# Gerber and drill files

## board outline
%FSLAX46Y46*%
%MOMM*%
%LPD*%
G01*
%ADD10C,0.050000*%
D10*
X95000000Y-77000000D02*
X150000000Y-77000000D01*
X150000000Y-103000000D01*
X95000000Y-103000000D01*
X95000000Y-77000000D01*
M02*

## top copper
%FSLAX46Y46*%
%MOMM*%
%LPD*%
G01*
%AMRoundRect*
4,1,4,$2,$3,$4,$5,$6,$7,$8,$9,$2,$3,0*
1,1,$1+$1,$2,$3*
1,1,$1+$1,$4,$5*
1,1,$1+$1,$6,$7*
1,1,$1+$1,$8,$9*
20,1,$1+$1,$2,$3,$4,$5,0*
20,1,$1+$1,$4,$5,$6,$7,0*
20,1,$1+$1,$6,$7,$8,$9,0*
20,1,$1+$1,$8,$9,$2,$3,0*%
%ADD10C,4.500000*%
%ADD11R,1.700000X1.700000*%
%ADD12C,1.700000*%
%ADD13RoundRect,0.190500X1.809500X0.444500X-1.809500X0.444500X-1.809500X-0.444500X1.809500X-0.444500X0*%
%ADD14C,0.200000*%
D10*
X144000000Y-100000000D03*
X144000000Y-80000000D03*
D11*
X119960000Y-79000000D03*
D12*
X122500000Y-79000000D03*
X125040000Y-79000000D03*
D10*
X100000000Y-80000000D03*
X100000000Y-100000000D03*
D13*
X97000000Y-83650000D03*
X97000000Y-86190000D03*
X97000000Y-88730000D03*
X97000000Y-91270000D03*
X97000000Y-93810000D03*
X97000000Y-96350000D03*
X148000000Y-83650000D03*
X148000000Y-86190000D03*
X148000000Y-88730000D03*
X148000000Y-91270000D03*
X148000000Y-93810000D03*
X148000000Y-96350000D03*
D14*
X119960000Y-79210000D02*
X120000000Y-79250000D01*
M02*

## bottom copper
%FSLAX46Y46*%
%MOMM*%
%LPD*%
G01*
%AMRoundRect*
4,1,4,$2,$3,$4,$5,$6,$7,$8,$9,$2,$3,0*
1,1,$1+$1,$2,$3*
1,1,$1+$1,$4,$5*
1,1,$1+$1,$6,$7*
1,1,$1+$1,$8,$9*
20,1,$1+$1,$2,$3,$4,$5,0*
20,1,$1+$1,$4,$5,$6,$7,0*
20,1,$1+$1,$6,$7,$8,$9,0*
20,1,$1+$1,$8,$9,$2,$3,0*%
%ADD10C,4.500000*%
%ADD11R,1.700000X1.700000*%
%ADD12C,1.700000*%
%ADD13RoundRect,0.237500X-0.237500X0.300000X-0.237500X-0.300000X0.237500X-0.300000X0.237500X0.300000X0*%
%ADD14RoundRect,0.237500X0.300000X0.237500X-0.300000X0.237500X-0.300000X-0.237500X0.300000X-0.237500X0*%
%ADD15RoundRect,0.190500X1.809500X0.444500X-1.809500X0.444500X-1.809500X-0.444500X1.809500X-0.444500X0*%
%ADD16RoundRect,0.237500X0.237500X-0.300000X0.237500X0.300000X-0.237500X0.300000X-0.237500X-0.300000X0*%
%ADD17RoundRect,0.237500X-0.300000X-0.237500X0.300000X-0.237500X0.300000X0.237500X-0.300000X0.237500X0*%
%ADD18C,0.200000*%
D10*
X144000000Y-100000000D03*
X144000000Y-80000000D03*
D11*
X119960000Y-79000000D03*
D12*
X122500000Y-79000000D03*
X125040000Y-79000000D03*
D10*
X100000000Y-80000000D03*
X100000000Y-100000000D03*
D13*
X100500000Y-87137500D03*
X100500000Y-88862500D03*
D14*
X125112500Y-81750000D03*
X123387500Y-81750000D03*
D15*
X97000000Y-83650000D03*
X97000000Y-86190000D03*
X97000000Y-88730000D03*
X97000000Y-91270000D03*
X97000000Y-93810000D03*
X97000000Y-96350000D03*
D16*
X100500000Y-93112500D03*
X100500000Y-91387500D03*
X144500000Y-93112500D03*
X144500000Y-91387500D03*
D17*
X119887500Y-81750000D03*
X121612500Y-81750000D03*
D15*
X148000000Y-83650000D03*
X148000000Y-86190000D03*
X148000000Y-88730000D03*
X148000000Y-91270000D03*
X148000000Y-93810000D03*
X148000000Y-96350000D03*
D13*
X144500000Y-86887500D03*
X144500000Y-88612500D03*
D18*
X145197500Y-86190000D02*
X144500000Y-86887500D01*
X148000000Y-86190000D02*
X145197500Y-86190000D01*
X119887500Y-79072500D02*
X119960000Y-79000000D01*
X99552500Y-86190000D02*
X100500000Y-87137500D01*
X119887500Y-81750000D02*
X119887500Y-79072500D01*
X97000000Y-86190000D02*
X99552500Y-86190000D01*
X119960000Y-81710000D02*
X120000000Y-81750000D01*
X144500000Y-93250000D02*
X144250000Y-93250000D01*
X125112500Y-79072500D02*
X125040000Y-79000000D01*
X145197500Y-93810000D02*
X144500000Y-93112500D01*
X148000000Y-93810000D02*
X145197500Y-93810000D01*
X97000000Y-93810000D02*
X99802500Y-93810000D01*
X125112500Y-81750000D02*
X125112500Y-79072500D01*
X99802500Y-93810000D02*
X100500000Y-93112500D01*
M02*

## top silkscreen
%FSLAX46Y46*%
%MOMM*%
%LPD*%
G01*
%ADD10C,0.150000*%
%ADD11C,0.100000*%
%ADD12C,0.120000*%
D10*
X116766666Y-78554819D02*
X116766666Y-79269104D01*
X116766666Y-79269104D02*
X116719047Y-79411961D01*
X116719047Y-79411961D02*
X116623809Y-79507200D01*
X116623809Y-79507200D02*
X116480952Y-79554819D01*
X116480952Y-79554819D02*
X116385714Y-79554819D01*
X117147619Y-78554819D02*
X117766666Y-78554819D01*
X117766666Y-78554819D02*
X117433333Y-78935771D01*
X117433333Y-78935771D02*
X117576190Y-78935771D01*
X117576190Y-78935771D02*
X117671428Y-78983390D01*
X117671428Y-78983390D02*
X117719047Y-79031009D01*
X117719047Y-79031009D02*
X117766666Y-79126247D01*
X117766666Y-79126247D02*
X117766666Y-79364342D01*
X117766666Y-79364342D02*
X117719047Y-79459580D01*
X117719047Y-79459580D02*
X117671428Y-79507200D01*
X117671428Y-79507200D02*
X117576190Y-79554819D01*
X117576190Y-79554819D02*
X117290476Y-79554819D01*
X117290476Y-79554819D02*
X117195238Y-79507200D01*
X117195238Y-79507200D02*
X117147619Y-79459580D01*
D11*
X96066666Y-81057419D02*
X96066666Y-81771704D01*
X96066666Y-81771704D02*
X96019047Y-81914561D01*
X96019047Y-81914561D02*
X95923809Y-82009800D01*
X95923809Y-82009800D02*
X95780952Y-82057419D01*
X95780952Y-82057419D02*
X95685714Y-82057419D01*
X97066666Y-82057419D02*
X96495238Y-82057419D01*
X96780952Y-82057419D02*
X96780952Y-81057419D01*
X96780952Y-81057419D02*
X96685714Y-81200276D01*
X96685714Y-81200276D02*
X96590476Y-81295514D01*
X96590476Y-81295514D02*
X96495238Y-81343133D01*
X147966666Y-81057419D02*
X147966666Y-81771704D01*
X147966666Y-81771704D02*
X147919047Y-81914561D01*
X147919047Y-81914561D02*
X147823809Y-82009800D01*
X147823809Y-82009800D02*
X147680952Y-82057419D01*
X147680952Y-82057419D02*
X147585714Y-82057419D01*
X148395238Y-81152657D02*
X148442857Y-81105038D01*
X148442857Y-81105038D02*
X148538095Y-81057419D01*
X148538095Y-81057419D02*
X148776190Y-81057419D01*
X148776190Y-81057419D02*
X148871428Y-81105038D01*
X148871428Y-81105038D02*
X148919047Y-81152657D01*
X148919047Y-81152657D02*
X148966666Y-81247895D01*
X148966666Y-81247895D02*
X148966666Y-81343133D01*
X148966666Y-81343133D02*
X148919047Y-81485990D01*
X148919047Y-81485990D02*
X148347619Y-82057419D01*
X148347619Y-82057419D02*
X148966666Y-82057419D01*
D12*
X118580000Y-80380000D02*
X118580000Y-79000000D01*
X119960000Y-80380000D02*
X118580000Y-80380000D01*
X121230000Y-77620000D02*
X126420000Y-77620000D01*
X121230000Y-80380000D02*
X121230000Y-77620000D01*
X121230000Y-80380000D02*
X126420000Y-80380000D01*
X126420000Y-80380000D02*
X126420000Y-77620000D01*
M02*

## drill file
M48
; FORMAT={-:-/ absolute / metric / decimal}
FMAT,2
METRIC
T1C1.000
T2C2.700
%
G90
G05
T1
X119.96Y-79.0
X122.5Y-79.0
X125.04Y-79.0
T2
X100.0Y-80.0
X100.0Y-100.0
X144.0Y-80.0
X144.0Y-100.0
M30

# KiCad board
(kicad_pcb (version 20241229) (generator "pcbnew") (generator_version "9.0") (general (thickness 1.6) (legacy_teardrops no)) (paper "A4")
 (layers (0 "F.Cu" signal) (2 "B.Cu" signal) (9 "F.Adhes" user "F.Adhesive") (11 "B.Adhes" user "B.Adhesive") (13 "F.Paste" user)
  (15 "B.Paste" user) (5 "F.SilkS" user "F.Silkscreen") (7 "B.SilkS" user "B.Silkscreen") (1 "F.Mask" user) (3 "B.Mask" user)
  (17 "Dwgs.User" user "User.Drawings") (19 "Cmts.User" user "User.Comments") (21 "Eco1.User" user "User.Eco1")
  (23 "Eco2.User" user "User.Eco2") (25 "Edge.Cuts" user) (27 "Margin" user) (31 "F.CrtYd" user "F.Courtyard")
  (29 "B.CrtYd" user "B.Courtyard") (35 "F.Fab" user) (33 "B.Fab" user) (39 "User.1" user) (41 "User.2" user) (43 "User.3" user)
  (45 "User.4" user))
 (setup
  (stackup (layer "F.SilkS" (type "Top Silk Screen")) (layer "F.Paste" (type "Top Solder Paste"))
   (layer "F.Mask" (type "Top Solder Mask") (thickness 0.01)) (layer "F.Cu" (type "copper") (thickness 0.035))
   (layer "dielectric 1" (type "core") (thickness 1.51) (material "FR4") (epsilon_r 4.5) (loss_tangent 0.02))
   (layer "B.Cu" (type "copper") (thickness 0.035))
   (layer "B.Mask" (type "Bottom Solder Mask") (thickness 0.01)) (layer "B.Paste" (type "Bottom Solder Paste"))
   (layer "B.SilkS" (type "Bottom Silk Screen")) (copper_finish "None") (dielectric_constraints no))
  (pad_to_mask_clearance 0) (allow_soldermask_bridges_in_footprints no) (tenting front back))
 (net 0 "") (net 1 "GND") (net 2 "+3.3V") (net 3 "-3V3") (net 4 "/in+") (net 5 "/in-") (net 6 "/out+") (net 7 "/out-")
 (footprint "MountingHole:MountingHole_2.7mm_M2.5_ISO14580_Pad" (layer "F.Cu") (at 144 100)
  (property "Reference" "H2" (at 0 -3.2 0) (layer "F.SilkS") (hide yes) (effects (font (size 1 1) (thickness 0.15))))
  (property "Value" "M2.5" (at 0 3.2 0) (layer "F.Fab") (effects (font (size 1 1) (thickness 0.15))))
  (pad "1" thru_hole circle (at 0 0) (size 4.5 4.5) (drill 2.7) (layers "*.Cu" "*.Mask") (remove_unused_layers no) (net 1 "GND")
   (zone_connect 2)))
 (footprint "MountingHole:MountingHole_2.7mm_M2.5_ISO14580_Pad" (layer "F.Cu") (at 144 80)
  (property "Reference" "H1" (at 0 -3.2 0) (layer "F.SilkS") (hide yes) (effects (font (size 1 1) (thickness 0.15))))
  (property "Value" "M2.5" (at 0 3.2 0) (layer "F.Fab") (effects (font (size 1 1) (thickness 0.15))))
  (pad "1" thru_hole circle (at 0 0) (size 4.5 4.5) (drill 2.7) (layers "*.Cu" "*.Mask") (remove_unused_layers no) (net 1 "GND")
   (zone_connect 2)))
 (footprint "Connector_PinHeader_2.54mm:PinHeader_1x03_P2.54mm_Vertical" (layer "F.Cu") (at 119.96 79 90)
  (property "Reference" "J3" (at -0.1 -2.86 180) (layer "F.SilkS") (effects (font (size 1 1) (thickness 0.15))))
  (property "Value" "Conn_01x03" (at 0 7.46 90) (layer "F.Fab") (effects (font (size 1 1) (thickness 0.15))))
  (fp_line (start -1.38 -1.38) (end 0 -1.38) (stroke (width 0.12) (type solid)) (layer "F.SilkS"))
  (fp_line (start -1.38 0) (end -1.38 -1.38) (stroke (width 0.12) (type solid)) (layer "F.SilkS"))
  (fp_line (start 1.38 1.27) (end 1.38 6.46) (stroke (width 0.12) (type solid)) (layer "F.SilkS"))
  (fp_line (start -1.38 1.27) (end 1.38 1.27) (stroke (width 0.12) (type solid)) (layer "F.SilkS"))
  (fp_line (start -1.38 1.27) (end -1.38 6.46) (stroke (width 0.12) (type solid)) (layer "F.SilkS"))
  (fp_line (start -1.38 6.46) (end 1.38 6.46) (stroke (width 0.12) (type solid)) (layer "F.SilkS"))
  (pad "1" thru_hole rect (at 0 0 90) (size 1.7 1.7) (drill 1) (layers "*.Cu" "*.Mask") (remove_unused_layers no) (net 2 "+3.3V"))
  (pad "2" thru_hole circle (at 0 2.54 90) (size 1.7 1.7) (drill 1) (layers "*.Cu" "*.Mask") (remove_unused_layers no) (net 1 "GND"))
  (pad "3" thru_hole circle (at 0 5.08 90) (size 1.7 1.7) (drill 1) (layers "*.Cu" "*.Mask") (remove_unused_layers no) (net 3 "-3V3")))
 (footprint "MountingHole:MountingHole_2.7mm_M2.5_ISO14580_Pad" (layer "F.Cu") (at 100 80)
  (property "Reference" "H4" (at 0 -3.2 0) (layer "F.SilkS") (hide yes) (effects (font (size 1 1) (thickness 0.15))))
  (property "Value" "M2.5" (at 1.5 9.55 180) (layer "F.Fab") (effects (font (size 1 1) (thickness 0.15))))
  (pad "1" thru_hole circle (at 0 0) (size 4.5 4.5) (drill 2.7) (layers "*.Cu" "*.Mask") (remove_unused_layers no) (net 1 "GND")
   (zone_connect 2)))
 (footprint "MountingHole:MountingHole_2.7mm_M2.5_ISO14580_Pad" (layer "F.Cu") (at 100 100)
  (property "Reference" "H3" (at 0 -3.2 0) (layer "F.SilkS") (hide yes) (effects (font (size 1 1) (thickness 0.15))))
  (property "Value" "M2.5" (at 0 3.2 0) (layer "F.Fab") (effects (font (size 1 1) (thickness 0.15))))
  (pad "1" thru_hole circle (at 0 0) (size 4.5 4.5) (drill 2.7) (layers "*.Cu" "*.Mask") (remove_unused_layers no) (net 1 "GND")
   (zone_connect 2)))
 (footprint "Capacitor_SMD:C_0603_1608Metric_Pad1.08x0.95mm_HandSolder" (layer "B.Cu") (at 100.5 88 -90)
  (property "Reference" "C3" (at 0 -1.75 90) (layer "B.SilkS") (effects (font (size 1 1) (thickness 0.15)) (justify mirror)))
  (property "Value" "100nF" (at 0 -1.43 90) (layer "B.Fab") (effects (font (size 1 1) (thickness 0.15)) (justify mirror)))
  (pad "1" smd roundrect (at -0.8625 0 270) (size 1.075 0.95) (layers "B.Cu" "B.Mask" "B.Paste") (roundrect_rratio 0.25) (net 2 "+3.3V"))
  (pad "2" smd roundrect (at 0.8625 0 270) (size 1.075 0.95) (layers "B.Cu" "B.Mask" "B.Paste") (roundrect_rratio 0.25) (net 1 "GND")))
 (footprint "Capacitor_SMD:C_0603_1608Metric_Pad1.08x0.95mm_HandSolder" (layer "B.Cu") (at 124.25 81.75 180)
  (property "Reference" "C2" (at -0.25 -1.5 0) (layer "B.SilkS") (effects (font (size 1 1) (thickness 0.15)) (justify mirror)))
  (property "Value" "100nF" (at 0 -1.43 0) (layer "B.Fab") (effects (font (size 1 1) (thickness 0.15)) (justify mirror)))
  (pad "1" smd roundrect (at -0.8625 0 180) (size 1.075 0.95) (layers "B.Cu" "B.Mask" "B.Paste") (roundrect_rratio 0.25) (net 3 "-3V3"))
  (pad "2" smd roundrect (at 0.8625 0 180) (size 1.075 0.95) (layers "B.Cu" "B.Mask" "B.Paste") (roundrect_rratio 0.25) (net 1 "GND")))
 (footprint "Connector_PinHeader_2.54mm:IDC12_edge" (layer "B.Cu") (at 97 83.65 180)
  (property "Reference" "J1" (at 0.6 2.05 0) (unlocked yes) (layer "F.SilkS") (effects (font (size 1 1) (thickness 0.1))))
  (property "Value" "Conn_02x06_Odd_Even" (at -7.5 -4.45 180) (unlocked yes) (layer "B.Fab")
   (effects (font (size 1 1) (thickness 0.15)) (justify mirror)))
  (pad "1" smd roundrect (at 0 0 180) (size 4 1.27) (layers "B.Cu" "B.Mask" "B.Paste") (roundrect_rratio 0.15) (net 1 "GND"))
  (pad "2" smd roundrect (at 0 0 180) (size 4 1.27) (layers "F.Cu" "F.Mask" "F.Paste") (roundrect_rratio 0.15) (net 1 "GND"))
  (pad "3" smd roundrect (at 0 -2.54 180) (size 4 1.27) (layers "B.Cu" "B.Mask" "B.Paste") (roundrect_rratio 0.15) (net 2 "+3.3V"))
  (pad "4" smd roundrect (at 0 -2.54 180) (size 4 1.27) (layers "F.Cu" "F.Mask" "F.Paste") (roundrect_rratio 0.15) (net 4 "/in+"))
  (pad "5" smd roundrect (at 0 -5.08 180) (size 4 1.27) (layers "B.Cu" "B.Mask" "B.Paste") (roundrect_rratio 0.15) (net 1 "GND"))
  (pad "6" smd roundrect (at 0 -5.08 180) (size 4 1.27) (layers "F.Cu" "F.Mask" "F.Paste") (roundrect_rratio 0.15) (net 1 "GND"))
  (pad "7" smd roundrect (at 0 -7.62 180) (size 4 1.27) (layers "B.Cu" "B.Mask" "B.Paste") (roundrect_rratio 0.15) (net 1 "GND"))
  (pad "8" smd roundrect (at 0 -7.62 180) (size 4 1.27) (layers "F.Cu" "F.Mask" "F.Paste") (roundrect_rratio 0.15) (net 1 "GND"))
  (pad "9" smd roundrect (at 0 -10.16 180) (size 4 1.27) (layers "B.Cu" "B.Mask" "B.Paste") (roundrect_rratio 0.15) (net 3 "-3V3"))
  (pad "10" smd roundrect (at 0 -10.16 180) (size 4 1.27) (layers "F.Cu" "F.Mask" "F.Paste") (roundrect_rratio 0.15) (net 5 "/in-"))
  (pad "11" smd roundrect (at 0 -12.7 180) (size 4 1.27) (layers "B.Cu" "B.Mask" "B.Paste") (roundrect_rratio 0.15) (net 1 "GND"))
  (pad "12" smd roundrect (at 0 -12.7 180) (size 4 1.27) (layers "F.Cu" "F.Mask" "F.Paste") (roundrect_rratio 0.15) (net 1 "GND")))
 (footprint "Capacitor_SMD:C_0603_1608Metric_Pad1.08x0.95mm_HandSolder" (layer "B.Cu") (at 100.5 92.25 90)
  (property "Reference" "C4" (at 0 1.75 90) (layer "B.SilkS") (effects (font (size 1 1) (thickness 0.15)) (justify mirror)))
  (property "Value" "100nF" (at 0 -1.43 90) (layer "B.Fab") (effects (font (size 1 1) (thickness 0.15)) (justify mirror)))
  (pad "1" smd roundrect (at -0.8625 0 90) (size 1.075 0.95) (layers "B.Cu" "B.Mask" "B.Paste") (roundrect_rratio 0.25) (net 3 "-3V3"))
  (pad "2" smd roundrect (at 0.8625 0 90) (size 1.075 0.95) (layers "B.Cu" "B.Mask" "B.Paste") (roundrect_rratio 0.25) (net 1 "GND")))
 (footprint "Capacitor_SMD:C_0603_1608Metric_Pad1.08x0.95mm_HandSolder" (layer "B.Cu") (at 144.5 92.25 90)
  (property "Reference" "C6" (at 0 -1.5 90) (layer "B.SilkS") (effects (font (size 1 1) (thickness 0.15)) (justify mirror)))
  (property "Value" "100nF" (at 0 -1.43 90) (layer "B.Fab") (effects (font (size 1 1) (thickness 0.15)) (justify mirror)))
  (pad "1" smd roundrect (at -0.8625 0 90) (size 1.075 0.95) (layers "B.Cu" "B.Mask" "B.Paste") (roundrect_rratio 0.25) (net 3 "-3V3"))
  (pad "2" smd roundrect (at 0.8625 0 90) (size 1.075 0.95) (layers "B.Cu" "B.Mask" "B.Paste") (roundrect_rratio 0.25) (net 1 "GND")))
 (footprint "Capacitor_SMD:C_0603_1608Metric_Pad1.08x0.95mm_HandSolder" (layer "B.Cu") (at 120.75 81.75)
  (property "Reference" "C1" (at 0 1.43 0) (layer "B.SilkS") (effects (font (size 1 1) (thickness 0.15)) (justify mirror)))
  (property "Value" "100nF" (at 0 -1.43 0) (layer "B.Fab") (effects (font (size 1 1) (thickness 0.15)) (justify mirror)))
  (pad "1" smd roundrect (at -0.8625 0) (size 1.075 0.95) (layers "B.Cu" "B.Mask" "B.Paste") (roundrect_rratio 0.25) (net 2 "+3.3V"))
  (pad "2" smd roundrect (at 0.8625 0) (size 1.075 0.95) (layers "B.Cu" "B.Mask" "B.Paste") (roundrect_rratio 0.25) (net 1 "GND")))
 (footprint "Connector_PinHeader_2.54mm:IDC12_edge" (layer "B.Cu") (at 148 83.65 180)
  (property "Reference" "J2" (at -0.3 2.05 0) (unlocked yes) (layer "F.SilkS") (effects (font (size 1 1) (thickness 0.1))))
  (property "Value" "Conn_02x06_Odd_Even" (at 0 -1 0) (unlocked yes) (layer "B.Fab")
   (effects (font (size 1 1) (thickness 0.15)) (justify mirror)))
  (pad "1" smd roundrect (at 0 0 180) (size 4 1.27) (layers "B.Cu" "B.Mask" "B.Paste") (roundrect_rratio 0.15) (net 1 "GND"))
  (pad "2" smd roundrect (at 0 0 180) (size 4 1.27) (layers "F.Cu" "F.Mask" "F.Paste") (roundrect_rratio 0.15) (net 1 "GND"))
  (pad "3" smd roundrect (at 0 -2.54 180) (size 4 1.27) (layers "B.Cu" "B.Mask" "B.Paste") (roundrect_rratio 0.15) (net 2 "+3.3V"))
  (pad "4" smd roundrect (at 0 -2.54 180) (size 4 1.27) (layers "F.Cu" "F.Mask" "F.Paste") (roundrect_rratio 0.15) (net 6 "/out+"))
  (pad "5" smd roundrect (at 0 -5.08 180) (size 4 1.27) (layers "B.Cu" "B.Mask" "B.Paste") (roundrect_rratio 0.15) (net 1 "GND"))
  (pad "6" smd roundrect (at 0 -5.08 180) (size 4 1.27) (layers "F.Cu" "F.Mask" "F.Paste") (roundrect_rratio 0.15) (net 1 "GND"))
  (pad "7" smd roundrect (at 0 -7.62 180) (size 4 1.27) (layers "B.Cu" "B.Mask" "B.Paste") (roundrect_rratio 0.15) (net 1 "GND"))
  (pad "8" smd roundrect (at 0 -7.62 180) (size 4 1.27) (layers "F.Cu" "F.Mask" "F.Paste") (roundrect_rratio 0.15) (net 1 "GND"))
  (pad "9" smd roundrect (at 0 -10.16 180) (size 4 1.27) (layers "B.Cu" "B.Mask" "B.Paste") (roundrect_rratio 0.15) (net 3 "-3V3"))
  (pad "10" smd roundrect (at 0 -10.16 180) (size 4 1.27) (layers "F.Cu" "F.Mask" "F.Paste") (roundrect_rratio 0.15) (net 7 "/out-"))
  (pad "11" smd roundrect (at 0 -12.7 180) (size 4 1.27) (layers "B.Cu" "B.Mask" "B.Paste") (roundrect_rratio 0.15) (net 1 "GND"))
  (pad "12" smd roundrect (at 0 -12.7 180) (size 4 1.27) (layers "F.Cu" "F.Mask" "F.Paste") (roundrect_rratio 0.15) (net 1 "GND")))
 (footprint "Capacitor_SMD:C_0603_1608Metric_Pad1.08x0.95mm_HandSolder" (layer "B.Cu") (at 144.5 87.75 -90)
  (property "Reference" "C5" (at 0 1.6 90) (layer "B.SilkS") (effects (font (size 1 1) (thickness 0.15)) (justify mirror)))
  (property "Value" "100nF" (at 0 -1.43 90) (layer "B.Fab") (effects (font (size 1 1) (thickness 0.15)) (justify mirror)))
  (pad "1" smd roundrect (at -0.8625 0 270) (size 1.075 0.95) (layers "B.Cu" "B.Mask" "B.Paste") (roundrect_rratio 0.25) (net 2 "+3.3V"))
  (pad "2" smd roundrect (at 0.8625 0 270) (size 1.075 0.95) (layers "B.Cu" "B.Mask" "B.Paste") (roundrect_rratio 0.25) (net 1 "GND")))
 (gr_rect (start 95 77) (end 150 103) (stroke (width 0.05) (type default)) (fill no) (layer "Edge.Cuts"))
 (segment (start 119.96 79.21) (end 120 79.25) (width 0.2) (layer "F.Cu") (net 2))
 (segment (start 145.1975 86.19) (end 144.5 86.8875) (width 0.2) (layer "B.Cu") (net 2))
 (segment (start 148 86.19) (end 145.1975 86.19) (width 0.2) (layer "B.Cu") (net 2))
 (segment (start 119.8875 79.0725) (end 119.96 79) (width 0.2) (layer "B.Cu") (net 2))
 (segment (start 99.5525 86.19) (end 100.5 87.1375) (width 0.2) (layer "B.Cu") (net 2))
 (segment (start 119.8875 81.75) (end 119.8875 79.0725) (width 0.2) (layer "B.Cu") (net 2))
 (segment (start 97 86.19) (end 99.5525 86.19) (width 0.2) (layer "B.Cu") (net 2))
 (segment (start 119.96 81.71) (end 120 81.75) (width 0.2) (layer "B.Cu") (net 2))
 (segment (start 144.5 93.25) (end 144.25 93.25) (width 0.2) (layer "B.Cu") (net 3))
 (segment (start 125.1125 79.0725) (end 125.04 79) (width 0.2) (layer "B.Cu") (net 3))
 (segment (start 145.1975 93.81) (end 144.5 93.1125) (width 0.2) (layer "B.Cu") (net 3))
 (segment (start 148 93.81) (end 145.1975 93.81) (width 0.2) (layer "B.Cu") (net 3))
 (segment (start 97 93.81) (end 99.8025 93.81) (width 0.2) (layer "B.Cu") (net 3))
 (segment (start 125.1125 81.75) (end 125.1125 79.0725) (width 0.2) (layer "B.Cu") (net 3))
 (segment (start 99.8025 93.81) (end 100.5 93.1125) (width 0.2) (layer "B.Cu") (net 3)))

